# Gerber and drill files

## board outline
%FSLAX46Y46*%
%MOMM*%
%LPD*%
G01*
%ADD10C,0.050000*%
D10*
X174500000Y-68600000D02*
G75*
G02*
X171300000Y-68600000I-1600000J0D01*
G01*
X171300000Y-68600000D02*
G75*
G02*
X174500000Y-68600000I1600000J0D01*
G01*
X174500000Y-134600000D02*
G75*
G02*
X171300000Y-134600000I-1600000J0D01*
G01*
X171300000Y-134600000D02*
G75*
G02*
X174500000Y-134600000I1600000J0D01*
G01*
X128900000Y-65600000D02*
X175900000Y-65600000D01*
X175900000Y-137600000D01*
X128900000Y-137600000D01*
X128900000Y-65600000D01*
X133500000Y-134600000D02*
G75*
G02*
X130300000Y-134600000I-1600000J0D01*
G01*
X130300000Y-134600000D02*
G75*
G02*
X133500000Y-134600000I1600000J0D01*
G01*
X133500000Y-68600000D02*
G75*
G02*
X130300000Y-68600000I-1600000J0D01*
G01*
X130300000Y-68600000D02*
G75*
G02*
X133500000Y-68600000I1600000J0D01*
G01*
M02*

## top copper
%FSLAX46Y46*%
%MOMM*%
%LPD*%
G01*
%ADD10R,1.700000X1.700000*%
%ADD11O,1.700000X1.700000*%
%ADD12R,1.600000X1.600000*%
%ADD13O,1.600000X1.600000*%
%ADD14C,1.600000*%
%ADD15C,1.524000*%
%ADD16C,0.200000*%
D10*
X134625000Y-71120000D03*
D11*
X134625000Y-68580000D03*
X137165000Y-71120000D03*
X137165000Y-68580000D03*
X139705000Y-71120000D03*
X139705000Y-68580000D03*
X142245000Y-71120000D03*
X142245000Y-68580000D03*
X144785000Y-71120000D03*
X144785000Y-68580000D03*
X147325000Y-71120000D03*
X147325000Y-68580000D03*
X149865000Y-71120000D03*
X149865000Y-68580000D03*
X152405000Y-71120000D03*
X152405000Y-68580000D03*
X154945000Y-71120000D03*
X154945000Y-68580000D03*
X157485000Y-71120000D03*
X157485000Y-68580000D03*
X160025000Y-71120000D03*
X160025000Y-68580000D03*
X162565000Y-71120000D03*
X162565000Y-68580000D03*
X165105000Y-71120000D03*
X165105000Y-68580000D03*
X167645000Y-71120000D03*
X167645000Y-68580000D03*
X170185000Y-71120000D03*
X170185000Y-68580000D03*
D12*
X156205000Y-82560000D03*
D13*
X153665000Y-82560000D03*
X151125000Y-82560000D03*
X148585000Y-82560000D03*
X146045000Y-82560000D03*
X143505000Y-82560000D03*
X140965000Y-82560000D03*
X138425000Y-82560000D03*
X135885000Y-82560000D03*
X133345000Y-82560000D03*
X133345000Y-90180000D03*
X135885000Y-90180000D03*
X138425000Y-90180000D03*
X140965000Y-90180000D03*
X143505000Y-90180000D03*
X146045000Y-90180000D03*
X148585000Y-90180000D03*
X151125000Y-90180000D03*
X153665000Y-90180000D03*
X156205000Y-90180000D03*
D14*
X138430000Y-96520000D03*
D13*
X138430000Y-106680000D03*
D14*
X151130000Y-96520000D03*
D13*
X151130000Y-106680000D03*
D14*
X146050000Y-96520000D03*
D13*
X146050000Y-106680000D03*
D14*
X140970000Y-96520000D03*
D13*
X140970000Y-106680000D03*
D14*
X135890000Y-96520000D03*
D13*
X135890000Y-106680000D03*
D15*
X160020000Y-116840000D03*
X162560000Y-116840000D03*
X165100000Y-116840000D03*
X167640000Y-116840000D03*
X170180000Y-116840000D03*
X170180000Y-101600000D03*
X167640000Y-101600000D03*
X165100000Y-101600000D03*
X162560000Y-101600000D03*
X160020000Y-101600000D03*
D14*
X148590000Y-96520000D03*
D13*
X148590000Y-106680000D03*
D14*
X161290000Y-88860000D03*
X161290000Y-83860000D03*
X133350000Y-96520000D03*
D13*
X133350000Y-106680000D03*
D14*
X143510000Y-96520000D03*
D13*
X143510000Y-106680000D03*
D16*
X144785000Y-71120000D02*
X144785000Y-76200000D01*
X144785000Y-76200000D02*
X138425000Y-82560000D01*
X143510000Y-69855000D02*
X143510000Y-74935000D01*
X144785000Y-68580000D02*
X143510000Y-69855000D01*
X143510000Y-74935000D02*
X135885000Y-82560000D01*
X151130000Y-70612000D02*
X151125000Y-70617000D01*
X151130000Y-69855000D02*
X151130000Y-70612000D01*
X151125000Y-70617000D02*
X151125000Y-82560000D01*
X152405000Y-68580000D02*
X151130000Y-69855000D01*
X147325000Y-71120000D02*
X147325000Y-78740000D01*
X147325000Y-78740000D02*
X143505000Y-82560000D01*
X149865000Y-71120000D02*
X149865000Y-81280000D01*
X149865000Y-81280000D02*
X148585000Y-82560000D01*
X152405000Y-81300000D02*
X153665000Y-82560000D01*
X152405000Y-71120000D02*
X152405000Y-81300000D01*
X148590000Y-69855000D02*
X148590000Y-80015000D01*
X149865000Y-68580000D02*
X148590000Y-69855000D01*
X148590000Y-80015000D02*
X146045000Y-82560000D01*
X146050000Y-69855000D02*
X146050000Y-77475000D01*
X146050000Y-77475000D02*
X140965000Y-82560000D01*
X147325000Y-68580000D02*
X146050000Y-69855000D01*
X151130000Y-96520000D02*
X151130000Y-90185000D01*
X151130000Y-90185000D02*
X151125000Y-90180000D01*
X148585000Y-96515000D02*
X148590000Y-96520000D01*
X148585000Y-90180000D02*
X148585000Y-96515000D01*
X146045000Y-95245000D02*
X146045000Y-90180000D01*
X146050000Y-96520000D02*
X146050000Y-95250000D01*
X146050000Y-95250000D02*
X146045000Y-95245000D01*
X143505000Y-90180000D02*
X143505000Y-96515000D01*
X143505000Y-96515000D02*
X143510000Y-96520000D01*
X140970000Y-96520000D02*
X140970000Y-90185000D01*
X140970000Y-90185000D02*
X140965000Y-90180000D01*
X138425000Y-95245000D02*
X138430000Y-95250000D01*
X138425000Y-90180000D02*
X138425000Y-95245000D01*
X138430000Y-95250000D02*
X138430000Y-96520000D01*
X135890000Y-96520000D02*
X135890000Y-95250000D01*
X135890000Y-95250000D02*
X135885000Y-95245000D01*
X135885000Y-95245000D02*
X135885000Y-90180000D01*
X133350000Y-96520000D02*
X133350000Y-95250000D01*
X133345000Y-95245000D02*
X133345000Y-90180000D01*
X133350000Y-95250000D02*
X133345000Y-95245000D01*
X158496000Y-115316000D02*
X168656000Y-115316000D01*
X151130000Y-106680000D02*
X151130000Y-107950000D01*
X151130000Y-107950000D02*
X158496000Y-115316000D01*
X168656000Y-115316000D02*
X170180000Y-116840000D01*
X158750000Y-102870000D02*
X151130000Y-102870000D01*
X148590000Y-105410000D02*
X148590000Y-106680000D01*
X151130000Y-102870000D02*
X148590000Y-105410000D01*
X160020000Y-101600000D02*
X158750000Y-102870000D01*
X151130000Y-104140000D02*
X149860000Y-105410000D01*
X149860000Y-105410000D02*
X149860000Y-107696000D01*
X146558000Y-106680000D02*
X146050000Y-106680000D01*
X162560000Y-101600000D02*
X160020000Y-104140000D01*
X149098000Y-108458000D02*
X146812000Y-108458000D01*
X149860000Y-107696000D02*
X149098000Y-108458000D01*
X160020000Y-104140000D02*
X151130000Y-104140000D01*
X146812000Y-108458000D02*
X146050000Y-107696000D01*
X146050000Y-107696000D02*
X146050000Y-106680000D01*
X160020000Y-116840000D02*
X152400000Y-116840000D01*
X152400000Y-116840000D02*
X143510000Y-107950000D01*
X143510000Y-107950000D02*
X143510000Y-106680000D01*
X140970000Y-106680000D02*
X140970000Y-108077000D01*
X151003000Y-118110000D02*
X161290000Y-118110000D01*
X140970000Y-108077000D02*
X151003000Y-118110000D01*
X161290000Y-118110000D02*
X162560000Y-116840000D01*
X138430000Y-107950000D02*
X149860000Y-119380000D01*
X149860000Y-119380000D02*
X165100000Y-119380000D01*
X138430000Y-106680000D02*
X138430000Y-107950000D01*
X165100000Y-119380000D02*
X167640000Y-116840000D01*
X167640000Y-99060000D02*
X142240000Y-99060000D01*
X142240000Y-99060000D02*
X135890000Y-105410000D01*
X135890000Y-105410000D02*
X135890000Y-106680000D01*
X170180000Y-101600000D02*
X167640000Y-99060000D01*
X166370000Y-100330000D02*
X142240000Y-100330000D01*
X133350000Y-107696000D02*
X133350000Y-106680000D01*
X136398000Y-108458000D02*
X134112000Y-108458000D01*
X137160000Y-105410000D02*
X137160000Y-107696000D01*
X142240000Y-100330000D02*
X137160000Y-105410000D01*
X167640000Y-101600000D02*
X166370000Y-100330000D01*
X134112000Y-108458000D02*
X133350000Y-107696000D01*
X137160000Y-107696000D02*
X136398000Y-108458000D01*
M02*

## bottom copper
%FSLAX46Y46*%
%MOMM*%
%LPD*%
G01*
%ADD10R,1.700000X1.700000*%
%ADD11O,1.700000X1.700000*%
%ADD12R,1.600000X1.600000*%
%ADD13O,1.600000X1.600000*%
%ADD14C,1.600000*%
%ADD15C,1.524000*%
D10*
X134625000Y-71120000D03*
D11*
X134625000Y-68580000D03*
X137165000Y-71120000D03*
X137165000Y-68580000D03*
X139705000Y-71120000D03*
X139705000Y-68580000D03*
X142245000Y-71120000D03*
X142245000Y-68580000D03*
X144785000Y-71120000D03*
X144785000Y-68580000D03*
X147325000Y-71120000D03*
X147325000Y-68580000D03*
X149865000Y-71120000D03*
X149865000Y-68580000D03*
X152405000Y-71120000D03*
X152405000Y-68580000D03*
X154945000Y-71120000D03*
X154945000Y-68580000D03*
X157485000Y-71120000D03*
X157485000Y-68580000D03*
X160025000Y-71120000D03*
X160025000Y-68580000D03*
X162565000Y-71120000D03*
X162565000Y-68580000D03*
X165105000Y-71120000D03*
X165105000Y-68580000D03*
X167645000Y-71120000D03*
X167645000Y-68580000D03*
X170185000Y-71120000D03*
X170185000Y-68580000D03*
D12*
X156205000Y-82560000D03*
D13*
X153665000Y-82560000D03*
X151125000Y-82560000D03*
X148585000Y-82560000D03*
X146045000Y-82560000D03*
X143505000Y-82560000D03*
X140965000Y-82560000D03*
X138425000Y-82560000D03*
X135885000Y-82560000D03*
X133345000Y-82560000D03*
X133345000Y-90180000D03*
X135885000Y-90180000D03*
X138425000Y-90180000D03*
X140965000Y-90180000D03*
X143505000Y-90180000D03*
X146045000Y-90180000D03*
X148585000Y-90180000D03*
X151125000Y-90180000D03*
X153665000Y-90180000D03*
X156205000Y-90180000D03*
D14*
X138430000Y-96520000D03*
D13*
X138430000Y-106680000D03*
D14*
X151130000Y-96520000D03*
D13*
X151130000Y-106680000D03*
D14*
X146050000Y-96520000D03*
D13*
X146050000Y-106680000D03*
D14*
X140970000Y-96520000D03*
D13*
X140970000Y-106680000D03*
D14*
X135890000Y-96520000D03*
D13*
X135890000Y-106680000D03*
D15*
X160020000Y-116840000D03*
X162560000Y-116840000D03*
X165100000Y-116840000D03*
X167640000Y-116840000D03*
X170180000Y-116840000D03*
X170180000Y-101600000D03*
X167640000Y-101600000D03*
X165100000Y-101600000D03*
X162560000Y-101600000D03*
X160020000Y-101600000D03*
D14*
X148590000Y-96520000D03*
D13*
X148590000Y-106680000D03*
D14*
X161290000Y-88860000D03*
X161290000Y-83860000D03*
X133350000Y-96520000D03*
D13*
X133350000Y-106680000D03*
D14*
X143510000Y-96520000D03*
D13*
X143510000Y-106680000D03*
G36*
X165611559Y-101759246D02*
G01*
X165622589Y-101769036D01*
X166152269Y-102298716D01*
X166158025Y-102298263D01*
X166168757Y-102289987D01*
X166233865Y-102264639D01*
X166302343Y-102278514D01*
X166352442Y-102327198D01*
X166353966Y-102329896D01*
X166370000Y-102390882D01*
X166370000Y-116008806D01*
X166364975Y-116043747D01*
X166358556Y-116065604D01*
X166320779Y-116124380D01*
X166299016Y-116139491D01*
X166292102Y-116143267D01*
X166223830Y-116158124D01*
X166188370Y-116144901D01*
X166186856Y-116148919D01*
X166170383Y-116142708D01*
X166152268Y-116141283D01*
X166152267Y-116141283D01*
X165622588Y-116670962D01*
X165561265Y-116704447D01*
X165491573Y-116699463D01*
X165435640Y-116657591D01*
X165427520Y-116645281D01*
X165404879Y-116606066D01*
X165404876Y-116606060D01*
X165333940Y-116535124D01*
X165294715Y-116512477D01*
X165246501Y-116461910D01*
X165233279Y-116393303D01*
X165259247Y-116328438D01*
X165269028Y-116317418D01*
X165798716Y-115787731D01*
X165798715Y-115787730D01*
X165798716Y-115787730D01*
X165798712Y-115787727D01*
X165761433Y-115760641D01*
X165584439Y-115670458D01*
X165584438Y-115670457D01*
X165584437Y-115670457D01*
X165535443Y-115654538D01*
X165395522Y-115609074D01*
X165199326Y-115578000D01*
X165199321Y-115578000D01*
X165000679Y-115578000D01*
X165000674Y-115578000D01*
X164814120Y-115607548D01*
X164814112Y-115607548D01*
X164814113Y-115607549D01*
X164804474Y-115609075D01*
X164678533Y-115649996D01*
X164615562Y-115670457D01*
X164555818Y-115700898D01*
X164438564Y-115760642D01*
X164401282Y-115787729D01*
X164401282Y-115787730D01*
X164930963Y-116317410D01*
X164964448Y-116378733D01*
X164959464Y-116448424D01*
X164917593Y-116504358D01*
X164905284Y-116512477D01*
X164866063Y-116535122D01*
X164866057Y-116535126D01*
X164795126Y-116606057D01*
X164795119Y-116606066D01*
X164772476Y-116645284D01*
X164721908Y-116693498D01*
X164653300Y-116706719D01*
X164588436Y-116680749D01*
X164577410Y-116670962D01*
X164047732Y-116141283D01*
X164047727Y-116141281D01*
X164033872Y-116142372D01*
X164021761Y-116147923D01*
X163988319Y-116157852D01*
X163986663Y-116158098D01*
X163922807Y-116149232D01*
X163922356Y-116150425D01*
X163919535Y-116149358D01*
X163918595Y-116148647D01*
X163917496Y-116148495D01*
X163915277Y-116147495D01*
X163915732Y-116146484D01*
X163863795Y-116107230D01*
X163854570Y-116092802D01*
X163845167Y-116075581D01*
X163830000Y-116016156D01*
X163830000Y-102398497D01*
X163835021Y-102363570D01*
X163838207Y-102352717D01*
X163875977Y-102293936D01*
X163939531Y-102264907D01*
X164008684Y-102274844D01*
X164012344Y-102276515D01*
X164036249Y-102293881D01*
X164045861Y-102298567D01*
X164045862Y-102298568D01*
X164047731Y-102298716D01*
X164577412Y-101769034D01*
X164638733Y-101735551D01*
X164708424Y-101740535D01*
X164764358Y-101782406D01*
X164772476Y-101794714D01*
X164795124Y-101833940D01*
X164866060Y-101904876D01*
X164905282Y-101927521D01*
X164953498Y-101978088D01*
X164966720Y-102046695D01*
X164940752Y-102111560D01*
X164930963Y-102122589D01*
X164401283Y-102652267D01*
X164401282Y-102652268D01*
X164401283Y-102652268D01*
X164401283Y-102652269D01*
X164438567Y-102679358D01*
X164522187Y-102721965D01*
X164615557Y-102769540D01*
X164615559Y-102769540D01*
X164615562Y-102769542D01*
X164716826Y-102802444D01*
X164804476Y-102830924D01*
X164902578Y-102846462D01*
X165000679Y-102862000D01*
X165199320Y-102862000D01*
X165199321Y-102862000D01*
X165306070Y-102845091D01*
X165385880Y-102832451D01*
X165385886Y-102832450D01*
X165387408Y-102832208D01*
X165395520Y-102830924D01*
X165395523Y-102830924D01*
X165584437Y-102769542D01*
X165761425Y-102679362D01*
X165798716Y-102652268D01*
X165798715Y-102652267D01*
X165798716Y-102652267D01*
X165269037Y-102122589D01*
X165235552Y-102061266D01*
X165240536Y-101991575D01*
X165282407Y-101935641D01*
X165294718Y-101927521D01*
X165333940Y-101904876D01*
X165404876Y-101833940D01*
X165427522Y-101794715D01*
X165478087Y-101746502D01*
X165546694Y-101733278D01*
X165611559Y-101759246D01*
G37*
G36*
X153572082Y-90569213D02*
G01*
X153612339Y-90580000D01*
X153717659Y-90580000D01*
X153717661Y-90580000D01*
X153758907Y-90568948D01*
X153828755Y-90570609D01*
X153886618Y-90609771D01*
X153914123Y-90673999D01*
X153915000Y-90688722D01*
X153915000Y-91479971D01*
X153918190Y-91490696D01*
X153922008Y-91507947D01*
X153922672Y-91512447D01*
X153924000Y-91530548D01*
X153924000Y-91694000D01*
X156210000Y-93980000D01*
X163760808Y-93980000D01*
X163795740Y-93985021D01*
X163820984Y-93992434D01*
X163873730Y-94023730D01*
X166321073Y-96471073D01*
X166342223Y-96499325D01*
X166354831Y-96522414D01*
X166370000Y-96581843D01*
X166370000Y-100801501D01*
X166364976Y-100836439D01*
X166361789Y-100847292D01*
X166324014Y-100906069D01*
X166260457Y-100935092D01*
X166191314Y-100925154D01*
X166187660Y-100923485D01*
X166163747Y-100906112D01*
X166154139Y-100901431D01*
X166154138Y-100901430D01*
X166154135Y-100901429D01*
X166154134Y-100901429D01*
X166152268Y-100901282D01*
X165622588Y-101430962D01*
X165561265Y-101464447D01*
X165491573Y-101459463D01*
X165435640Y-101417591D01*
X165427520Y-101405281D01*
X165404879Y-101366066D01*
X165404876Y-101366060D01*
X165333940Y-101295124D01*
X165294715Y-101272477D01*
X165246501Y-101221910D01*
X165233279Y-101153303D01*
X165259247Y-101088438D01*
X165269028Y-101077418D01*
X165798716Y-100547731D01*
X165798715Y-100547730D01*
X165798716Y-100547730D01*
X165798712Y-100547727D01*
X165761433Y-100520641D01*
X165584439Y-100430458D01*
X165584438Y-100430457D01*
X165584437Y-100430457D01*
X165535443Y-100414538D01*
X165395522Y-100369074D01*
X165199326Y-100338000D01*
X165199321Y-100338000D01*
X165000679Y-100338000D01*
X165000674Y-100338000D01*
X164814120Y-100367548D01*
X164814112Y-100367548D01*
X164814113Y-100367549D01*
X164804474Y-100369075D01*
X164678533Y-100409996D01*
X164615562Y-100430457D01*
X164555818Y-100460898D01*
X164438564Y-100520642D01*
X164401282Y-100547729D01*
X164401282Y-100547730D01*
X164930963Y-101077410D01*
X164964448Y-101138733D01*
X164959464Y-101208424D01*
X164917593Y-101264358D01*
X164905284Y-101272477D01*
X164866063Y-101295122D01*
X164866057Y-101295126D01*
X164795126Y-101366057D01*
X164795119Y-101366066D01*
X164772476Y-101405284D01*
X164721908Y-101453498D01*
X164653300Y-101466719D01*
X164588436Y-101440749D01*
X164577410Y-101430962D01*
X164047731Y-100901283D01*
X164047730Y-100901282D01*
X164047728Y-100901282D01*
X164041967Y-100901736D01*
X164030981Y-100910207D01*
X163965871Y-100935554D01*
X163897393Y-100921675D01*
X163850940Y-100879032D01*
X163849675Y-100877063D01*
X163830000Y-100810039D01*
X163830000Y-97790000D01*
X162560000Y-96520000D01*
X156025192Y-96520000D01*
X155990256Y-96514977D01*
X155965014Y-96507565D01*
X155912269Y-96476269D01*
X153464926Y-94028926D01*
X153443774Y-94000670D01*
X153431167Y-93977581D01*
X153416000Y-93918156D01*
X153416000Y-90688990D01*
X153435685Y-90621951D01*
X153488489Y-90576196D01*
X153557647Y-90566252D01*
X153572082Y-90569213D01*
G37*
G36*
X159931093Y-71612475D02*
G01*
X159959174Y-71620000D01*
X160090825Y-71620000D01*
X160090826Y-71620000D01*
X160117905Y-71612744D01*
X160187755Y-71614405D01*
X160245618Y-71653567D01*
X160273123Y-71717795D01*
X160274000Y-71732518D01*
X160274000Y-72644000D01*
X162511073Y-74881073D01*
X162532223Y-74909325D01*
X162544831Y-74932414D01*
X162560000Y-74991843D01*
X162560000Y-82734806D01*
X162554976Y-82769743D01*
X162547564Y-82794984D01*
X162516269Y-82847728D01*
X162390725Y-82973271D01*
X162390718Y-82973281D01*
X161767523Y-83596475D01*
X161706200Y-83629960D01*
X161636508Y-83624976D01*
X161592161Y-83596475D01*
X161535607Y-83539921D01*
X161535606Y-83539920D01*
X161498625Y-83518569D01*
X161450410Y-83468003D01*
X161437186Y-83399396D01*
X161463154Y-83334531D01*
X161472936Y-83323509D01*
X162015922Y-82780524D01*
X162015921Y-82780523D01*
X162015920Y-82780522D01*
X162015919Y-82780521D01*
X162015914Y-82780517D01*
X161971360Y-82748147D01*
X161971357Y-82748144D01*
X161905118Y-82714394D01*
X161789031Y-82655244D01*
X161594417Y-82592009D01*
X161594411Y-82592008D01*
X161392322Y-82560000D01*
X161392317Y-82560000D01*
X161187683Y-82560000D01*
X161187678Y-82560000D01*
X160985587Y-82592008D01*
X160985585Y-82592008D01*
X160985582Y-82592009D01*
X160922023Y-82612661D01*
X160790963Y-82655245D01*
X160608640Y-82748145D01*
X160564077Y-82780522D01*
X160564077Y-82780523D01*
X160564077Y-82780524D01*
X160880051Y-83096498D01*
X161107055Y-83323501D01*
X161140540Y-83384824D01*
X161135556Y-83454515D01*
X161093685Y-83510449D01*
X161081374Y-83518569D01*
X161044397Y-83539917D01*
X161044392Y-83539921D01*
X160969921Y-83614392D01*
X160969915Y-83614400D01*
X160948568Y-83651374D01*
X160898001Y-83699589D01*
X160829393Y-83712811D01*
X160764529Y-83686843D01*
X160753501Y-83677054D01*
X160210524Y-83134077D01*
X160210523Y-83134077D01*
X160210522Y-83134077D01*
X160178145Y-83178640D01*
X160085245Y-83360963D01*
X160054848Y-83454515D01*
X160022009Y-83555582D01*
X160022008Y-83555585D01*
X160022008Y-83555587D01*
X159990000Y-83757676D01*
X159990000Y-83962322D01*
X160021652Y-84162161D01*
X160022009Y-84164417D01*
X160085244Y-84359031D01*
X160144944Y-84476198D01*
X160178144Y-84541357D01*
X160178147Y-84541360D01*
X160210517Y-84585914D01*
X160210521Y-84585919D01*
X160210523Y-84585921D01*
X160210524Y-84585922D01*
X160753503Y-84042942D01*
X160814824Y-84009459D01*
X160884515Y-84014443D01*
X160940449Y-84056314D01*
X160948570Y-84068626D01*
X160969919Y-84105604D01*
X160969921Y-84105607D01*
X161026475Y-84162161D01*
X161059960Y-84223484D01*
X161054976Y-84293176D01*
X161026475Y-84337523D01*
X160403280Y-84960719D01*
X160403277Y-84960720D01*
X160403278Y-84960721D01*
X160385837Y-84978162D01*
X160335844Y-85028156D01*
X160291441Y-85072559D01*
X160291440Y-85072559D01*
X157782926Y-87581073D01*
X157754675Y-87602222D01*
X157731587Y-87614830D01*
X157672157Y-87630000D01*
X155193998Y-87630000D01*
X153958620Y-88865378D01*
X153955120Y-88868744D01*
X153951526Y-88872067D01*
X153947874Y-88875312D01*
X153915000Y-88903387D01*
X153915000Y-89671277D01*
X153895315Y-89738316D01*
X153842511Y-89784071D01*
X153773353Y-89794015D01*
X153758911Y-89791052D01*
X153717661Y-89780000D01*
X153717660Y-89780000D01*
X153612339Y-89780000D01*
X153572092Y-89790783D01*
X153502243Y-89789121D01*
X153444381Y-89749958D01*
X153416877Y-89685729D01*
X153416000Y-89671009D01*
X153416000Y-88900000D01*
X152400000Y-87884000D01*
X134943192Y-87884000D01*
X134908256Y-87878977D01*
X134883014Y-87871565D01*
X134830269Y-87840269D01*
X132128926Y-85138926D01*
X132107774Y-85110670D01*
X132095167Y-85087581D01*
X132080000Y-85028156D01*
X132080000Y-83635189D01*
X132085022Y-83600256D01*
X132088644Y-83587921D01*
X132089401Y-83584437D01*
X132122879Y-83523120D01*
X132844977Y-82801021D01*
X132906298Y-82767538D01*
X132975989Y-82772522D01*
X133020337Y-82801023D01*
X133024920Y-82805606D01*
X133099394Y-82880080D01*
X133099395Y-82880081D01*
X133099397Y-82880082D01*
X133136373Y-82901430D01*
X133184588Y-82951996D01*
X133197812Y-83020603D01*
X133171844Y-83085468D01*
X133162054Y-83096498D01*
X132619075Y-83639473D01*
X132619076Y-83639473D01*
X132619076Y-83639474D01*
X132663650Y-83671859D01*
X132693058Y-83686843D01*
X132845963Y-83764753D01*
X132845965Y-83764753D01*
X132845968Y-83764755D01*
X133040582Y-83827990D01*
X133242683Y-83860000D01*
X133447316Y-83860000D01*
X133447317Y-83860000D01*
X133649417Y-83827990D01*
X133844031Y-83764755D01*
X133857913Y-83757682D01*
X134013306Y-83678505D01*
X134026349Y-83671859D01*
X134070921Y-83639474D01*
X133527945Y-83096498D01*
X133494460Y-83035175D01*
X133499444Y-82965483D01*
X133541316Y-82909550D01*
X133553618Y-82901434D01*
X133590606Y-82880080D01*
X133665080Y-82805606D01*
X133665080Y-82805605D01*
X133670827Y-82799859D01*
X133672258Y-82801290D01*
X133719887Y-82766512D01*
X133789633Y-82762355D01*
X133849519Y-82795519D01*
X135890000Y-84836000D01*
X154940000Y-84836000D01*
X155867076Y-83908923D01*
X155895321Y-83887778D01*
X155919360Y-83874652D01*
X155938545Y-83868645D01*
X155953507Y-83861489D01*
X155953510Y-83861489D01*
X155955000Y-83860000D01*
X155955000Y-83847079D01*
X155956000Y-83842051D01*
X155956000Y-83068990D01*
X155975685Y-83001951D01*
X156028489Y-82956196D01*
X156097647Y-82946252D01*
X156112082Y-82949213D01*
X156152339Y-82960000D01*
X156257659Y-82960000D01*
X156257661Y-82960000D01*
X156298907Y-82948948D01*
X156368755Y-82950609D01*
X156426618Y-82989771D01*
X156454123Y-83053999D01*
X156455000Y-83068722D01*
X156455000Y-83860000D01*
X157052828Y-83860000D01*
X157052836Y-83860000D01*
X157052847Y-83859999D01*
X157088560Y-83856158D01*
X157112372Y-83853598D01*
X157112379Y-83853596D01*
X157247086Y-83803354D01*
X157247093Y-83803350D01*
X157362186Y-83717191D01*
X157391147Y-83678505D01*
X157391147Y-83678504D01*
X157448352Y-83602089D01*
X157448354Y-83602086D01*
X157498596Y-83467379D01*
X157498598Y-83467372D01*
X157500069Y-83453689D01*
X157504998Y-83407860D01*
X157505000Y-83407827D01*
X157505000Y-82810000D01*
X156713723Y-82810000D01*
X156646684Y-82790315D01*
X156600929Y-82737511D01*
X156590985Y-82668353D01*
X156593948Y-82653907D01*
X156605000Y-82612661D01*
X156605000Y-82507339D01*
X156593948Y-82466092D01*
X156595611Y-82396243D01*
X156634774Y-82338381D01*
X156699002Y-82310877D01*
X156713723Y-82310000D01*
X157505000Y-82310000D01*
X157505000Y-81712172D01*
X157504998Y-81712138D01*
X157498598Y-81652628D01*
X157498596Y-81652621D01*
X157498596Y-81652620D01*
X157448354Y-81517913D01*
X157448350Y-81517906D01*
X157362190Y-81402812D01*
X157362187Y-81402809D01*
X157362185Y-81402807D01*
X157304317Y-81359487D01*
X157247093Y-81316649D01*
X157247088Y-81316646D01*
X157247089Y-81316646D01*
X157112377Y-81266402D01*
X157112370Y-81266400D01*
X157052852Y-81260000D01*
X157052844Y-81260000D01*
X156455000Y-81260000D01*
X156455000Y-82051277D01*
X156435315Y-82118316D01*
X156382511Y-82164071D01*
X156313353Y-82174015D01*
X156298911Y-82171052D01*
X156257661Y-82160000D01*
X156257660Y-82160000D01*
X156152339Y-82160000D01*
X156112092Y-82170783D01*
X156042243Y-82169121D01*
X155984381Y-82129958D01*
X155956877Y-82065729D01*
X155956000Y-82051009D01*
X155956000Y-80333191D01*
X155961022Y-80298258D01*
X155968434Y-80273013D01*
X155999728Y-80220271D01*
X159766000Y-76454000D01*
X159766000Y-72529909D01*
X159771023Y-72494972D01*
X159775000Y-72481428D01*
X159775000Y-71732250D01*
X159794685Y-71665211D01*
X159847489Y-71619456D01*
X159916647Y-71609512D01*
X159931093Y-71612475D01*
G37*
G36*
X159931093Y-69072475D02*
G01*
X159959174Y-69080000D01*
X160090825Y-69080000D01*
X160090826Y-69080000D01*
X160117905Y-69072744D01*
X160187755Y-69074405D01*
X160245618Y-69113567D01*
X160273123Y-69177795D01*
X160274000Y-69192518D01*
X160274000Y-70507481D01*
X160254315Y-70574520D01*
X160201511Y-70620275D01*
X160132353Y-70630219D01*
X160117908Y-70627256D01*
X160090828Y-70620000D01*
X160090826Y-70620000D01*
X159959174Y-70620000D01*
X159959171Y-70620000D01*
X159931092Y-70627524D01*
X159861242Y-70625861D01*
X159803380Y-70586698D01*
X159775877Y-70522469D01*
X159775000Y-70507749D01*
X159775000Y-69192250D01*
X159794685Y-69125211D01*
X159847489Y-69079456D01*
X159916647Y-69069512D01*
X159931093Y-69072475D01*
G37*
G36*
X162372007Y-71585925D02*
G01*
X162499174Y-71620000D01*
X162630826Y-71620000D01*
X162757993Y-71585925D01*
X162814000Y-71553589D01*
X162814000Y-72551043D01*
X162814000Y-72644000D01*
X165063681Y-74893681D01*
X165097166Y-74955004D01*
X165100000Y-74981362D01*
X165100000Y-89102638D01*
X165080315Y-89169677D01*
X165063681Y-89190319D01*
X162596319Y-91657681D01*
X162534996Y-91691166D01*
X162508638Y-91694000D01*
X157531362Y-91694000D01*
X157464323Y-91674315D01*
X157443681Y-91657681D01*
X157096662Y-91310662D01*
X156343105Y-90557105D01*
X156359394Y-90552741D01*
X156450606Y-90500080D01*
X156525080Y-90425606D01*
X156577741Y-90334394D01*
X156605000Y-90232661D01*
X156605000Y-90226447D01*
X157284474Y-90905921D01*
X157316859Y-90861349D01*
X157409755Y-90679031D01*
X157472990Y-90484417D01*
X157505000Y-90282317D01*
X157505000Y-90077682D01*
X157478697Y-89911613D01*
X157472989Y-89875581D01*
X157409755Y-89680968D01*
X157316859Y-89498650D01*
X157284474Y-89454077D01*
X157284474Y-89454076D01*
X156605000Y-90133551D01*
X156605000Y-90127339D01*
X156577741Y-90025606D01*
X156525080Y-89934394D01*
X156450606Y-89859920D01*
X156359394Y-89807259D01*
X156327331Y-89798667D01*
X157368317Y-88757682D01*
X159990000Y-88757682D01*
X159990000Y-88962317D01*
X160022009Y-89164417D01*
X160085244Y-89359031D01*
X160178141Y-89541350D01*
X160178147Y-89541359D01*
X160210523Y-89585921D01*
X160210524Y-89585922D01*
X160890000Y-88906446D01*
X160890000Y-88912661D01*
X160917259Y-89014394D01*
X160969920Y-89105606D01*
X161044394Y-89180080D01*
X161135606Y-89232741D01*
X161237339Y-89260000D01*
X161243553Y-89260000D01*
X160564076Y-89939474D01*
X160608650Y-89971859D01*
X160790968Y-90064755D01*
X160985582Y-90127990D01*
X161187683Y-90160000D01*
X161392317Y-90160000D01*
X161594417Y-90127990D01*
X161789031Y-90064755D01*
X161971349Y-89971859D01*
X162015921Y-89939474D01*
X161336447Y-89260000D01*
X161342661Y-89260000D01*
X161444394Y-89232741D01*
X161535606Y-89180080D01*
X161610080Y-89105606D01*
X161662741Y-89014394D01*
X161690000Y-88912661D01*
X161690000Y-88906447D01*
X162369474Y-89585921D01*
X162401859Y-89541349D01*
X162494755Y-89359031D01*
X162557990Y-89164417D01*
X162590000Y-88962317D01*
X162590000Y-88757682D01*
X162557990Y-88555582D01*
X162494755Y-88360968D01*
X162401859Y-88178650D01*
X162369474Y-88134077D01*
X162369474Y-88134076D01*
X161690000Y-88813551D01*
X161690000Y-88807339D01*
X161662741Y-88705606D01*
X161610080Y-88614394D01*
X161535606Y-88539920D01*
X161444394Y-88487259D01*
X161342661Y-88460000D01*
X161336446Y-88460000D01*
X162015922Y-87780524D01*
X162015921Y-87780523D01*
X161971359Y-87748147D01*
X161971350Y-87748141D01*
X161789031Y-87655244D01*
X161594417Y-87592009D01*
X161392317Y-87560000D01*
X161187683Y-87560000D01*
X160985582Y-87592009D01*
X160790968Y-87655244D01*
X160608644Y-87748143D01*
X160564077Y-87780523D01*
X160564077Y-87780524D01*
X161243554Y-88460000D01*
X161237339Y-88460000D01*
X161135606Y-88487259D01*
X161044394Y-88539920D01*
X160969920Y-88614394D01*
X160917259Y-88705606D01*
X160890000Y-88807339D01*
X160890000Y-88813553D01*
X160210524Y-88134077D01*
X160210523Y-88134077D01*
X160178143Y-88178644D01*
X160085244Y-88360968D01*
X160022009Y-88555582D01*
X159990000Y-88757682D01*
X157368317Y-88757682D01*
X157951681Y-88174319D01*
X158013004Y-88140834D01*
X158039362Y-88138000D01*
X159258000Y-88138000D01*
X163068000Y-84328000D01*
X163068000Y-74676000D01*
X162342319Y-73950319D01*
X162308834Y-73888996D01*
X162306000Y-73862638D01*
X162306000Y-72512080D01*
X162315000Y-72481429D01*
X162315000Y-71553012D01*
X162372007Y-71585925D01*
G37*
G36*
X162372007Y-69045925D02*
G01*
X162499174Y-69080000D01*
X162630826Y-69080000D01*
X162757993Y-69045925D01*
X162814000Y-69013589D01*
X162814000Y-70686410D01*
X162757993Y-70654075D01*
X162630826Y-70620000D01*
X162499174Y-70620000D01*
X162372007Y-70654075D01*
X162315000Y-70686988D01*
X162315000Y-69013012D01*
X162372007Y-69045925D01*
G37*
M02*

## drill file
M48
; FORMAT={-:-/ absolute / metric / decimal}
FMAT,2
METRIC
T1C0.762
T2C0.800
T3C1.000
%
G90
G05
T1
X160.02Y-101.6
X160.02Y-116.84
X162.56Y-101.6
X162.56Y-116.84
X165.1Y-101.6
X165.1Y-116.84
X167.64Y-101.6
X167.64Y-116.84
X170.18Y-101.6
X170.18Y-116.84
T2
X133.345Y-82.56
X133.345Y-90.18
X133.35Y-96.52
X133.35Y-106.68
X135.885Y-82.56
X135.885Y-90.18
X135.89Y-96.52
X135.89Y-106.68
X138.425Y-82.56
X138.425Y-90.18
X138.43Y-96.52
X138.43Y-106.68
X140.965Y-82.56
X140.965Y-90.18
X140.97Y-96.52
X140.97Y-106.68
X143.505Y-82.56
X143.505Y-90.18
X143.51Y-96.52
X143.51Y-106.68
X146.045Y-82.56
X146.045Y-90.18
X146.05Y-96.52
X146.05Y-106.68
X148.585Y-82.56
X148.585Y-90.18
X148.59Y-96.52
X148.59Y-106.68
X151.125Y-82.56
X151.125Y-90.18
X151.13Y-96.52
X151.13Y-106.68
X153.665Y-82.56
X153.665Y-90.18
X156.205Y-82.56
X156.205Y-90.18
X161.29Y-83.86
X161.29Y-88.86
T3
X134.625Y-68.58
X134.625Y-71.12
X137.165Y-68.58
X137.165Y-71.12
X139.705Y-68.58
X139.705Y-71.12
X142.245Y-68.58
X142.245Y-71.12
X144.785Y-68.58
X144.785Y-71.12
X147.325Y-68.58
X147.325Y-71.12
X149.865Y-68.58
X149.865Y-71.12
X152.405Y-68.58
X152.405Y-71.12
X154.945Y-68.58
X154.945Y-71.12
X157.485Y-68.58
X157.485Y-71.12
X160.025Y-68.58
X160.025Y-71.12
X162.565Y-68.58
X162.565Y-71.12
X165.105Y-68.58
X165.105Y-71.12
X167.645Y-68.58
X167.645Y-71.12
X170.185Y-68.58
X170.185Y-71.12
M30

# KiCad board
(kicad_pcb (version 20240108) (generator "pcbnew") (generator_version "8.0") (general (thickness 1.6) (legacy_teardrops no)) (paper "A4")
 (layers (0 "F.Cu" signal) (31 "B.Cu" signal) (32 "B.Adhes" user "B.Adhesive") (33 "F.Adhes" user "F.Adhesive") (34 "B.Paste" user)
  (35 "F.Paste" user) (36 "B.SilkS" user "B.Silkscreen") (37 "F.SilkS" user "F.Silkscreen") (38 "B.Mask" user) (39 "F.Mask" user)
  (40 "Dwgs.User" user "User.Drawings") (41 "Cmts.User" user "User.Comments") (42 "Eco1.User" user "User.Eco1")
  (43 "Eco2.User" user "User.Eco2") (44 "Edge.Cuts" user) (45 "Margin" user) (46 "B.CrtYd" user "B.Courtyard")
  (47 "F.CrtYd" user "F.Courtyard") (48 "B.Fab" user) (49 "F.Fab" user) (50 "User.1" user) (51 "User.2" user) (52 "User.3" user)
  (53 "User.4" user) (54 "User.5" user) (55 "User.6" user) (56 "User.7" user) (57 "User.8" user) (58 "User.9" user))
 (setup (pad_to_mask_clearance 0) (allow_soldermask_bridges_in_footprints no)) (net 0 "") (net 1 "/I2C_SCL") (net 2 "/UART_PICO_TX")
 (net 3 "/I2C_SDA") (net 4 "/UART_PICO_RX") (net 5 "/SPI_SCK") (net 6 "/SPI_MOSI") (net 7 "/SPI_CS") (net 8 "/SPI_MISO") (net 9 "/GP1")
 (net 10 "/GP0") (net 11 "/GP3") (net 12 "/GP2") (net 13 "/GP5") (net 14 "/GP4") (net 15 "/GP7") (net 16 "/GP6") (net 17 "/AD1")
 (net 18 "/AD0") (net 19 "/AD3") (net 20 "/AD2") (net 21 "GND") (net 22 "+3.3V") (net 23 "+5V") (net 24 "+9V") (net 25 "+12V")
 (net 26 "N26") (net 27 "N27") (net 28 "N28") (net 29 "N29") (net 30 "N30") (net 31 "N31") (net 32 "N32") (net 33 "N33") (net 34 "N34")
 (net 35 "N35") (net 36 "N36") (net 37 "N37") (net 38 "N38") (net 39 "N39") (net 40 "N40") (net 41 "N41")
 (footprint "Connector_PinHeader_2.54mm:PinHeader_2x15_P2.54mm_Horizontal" (layer "F.Cu") (at 134.625 71.12 90)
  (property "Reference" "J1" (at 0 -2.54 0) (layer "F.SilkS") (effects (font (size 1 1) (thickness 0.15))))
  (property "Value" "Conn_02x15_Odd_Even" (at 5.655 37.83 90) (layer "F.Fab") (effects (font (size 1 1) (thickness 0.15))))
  (pad "1" thru_hole rect (at 0 0 90) (size 1.7 1.7) (drill 1) (layers "*.Cu" "*.Mask") (remove_unused_layers no) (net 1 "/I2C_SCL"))
  (pad "2" thru_hole oval (at 2.54 0 90) (size 1.7 1.7) (drill 1) (layers "*.Cu" "*.Mask") (remove_unused_layers no) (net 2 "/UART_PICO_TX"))
  (pad "3" thru_hole oval (at 0 2.54 90) (size 1.7 1.7) (drill 1) (layers "*.Cu" "*.Mask") (remove_unused_layers no) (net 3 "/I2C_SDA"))
  (pad "4" thru_hole oval (at 2.54 2.54 90) (size 1.7 1.7) (drill 1) (layers "*.Cu" "*.Mask") (remove_unused_layers no)
   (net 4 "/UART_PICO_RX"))
  (pad "5" thru_hole oval (at 0 5.08 90) (size 1.7 1.7) (drill 1) (layers "*.Cu" "*.Mask") (remove_unused_layers no) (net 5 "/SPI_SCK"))
  (pad "6" thru_hole oval (at 2.54 5.08 90) (size 1.7 1.7) (drill 1) (layers "*.Cu" "*.Mask") (remove_unused_layers no) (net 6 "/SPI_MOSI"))
  (pad "7" thru_hole oval (at 0 7.62 90) (size 1.7 1.7) (drill 1) (layers "*.Cu" "*.Mask") (remove_unused_layers no) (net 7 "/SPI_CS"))
  (pad "8" thru_hole oval (at 2.54 7.62 90) (size 1.7 1.7) (drill 1) (layers "*.Cu" "*.Mask") (remove_unused_layers no) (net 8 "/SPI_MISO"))
  (pad "9" thru_hole oval (at 0 10.16 90) (size 1.7 1.7) (drill 1) (layers "*.Cu" "*.Mask") (remove_unused_layers no) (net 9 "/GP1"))
  (pad "10" thru_hole oval (at 2.54 10.16 90) (size 1.7 1.7) (drill 1) (layers "*.Cu" "*.Mask") (remove_unused_layers no) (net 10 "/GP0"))
  (pad "11" thru_hole oval (at 0 12.7 90) (size 1.7 1.7) (drill 1) (layers "*.Cu" "*.Mask") (remove_unused_layers no) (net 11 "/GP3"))
  (pad "12" thru_hole oval (at 2.54 12.7 90) (size 1.7 1.7) (drill 1) (layers "*.Cu" "*.Mask") (remove_unused_layers no) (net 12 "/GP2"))
  (pad "13" thru_hole oval (at 0 15.24 90) (size 1.7 1.7) (drill 1) (layers "*.Cu" "*.Mask") (remove_unused_layers no) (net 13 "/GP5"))
  (pad "14" thru_hole oval (at 2.54 15.24 90) (size 1.7 1.7) (drill 1) (layers "*.Cu" "*.Mask") (remove_unused_layers no) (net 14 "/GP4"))
  (pad "15" thru_hole oval (at 0 17.78 90) (size 1.7 1.7) (drill 1) (layers "*.Cu" "*.Mask") (remove_unused_layers no) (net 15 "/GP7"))
  (pad "16" thru_hole oval (at 2.54 17.78 90) (size 1.7 1.7) (drill 1) (layers "*.Cu" "*.Mask") (remove_unused_layers no) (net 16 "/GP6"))
  (pad "17" thru_hole oval (at 0 20.32 90) (size 1.7 1.7) (drill 1) (layers "*.Cu" "*.Mask") (remove_unused_layers no) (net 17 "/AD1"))
  (pad "18" thru_hole oval (at 2.54 20.32 90) (size 1.7 1.7) (drill 1) (layers "*.Cu" "*.Mask") (remove_unused_layers no) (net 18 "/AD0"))
  (pad "19" thru_hole oval (at 0 22.86 90) (size 1.7 1.7) (drill 1) (layers "*.Cu" "*.Mask") (remove_unused_layers no) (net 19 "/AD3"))
  (pad "20" thru_hole oval (at 2.54 22.86 90) (size 1.7 1.7) (drill 1) (layers "*.Cu" "*.Mask") (remove_unused_layers no) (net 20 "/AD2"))
  (pad "21" thru_hole oval (at 0 25.4 90) (size 1.7 1.7) (drill 1) (layers "*.Cu" "*.Mask") (remove_unused_layers no) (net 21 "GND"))
  (pad "22" thru_hole oval (at 2.54 25.4 90) (size 1.7 1.7) (drill 1) (layers "*.Cu" "*.Mask") (remove_unused_layers no) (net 21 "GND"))
  (pad "23" thru_hole oval (at 0 27.94 90) (size 1.7 1.7) (drill 1) (layers "*.Cu" "*.Mask") (remove_unused_layers no) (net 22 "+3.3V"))
  (pad "24" thru_hole oval (at 2.54 27.94 90) (size 1.7 1.7) (drill 1) (layers "*.Cu" "*.Mask") (remove_unused_layers no) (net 22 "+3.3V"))
  (pad "25" thru_hole oval (at 0 30.48 90) (size 1.7 1.7) (drill 1) (layers "*.Cu" "*.Mask") (remove_unused_layers no) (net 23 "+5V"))
  (pad "26" thru_hole oval (at 2.54 30.48 90) (size 1.7 1.7) (drill 1) (layers "*.Cu" "*.Mask") (remove_unused_layers no) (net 23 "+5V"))
  (pad "27" thru_hole oval (at 0 33.02 90) (size 1.7 1.7) (drill 1) (layers "*.Cu" "*.Mask") (remove_unused_layers no) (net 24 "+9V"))
  (pad "28" thru_hole oval (at 2.54 33.02 90) (size 1.7 1.7) (drill 1) (layers "*.Cu" "*.Mask") (remove_unused_layers no) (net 24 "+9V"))
  (pad "29" thru_hole oval (at 0 35.56 90) (size 1.7 1.7) (drill 1) (layers "*.Cu" "*.Mask") (remove_unused_layers no) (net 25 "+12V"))
  (pad "30" thru_hole oval (at 2.54 35.56 90) (size 1.7 1.7) (drill 1) (layers "*.Cu" "*.Mask") (remove_unused_layers no) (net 25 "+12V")))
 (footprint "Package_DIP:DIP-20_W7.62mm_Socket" (layer "F.Cu") (at 156.205 82.56 -90)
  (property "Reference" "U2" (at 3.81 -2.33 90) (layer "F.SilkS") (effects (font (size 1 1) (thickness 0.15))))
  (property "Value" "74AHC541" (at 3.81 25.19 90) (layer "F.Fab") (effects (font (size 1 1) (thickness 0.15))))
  (pad "1" thru_hole rect (at 0 0 270) (size 1.6 1.6) (drill 0.8) (layers "*.Cu" "*.Mask") (remove_unused_layers no) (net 21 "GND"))
  (pad "2" thru_hole oval (at 0 2.54 270) (size 1.6 1.6) (drill 0.8) (layers "*.Cu" "*.Mask") (remove_unused_layers no) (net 15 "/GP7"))
  (pad "3" thru_hole oval (at 0 5.08 270) (size 1.6 1.6) (drill 0.8) (layers "*.Cu" "*.Mask") (remove_unused_layers no) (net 16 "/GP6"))
  (pad "4" thru_hole oval (at 0 7.62 270) (size 1.6 1.6) (drill 0.8) (layers "*.Cu" "*.Mask") (remove_unused_layers no) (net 13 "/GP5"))
  (pad "5" thru_hole oval (at 0 10.16 270) (size 1.6 1.6) (drill 0.8) (layers "*.Cu" "*.Mask") (remove_unused_layers no) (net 14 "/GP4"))
  (pad "6" thru_hole oval (at 0 12.7 270) (size 1.6 1.6) (drill 0.8) (layers "*.Cu" "*.Mask") (remove_unused_layers no) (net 11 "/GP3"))
  (pad "7" thru_hole oval (at 0 15.24 270) (size 1.6 1.6) (drill 0.8) (layers "*.Cu" "*.Mask") (remove_unused_layers no) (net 12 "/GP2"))
  (pad "8" thru_hole oval (at 0 17.78 270) (size 1.6 1.6) (drill 0.8) (layers "*.Cu" "*.Mask") (remove_unused_layers no) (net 9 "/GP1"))
  (pad "9" thru_hole oval (at 0 20.32 270) (size 1.6 1.6) (drill 0.8) (layers "*.Cu" "*.Mask") (remove_unused_layers no) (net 10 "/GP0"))
  (pad "10" thru_hole oval (at 0 22.86 270) (size 1.6 1.6) (drill 0.8) (layers "*.Cu" "*.Mask") (remove_unused_layers no) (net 21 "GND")
   (thermal_bridge_angle 45))
  (pad "11" thru_hole oval (at 7.62 22.86 270) (size 1.6 1.6) (drill 0.8) (layers "*.Cu" "*.Mask") (remove_unused_layers no) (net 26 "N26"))
  (pad "12" thru_hole oval (at 7.62 20.32 270) (size 1.6 1.6) (drill 0.8) (layers "*.Cu" "*.Mask") (remove_unused_layers no) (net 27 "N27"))
  (pad "13" thru_hole oval (at 7.62 17.78 270) (size 1.6 1.6) (drill 0.8) (layers "*.Cu" "*.Mask") (remove_unused_layers no) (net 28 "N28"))
  (pad "14" thru_hole oval (at 7.62 15.24 270) (size 1.6 1.6) (drill 0.8) (layers "*.Cu" "*.Mask") (remove_unused_layers no) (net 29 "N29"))
  (pad "15" thru_hole oval (at 7.62 12.7 270) (size 1.6 1.6) (drill 0.8) (layers "*.Cu" "*.Mask") (remove_unused_layers no) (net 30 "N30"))
  (pad "16" thru_hole oval (at 7.62 10.16 270) (size 1.6 1.6) (drill 0.8) (layers "*.Cu" "*.Mask") (remove_unused_layers no) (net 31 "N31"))
  (pad "17" thru_hole oval (at 7.62 7.62 270) (size 1.6 1.6) (drill 0.8) (layers "*.Cu" "*.Mask") (remove_unused_layers no) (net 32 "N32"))
  (pad "18" thru_hole oval (at 7.62 5.08 270) (size 1.6 1.6) (drill 0.8) (layers "*.Cu" "*.Mask") (remove_unused_layers no) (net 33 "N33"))
  (pad "19" thru_hole oval (at 7.62 2.54 270) (size 1.6 1.6) (drill 0.8) (layers "*.Cu" "*.Mask") (remove_unused_layers no) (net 21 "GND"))
  (pad "20" thru_hole oval (at 7.62 0 270) (size 1.6 1.6) (drill 0.8) (layers "*.Cu" "*.Mask") (remove_unused_layers no) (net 22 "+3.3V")
   (thermal_bridge_angle 45)))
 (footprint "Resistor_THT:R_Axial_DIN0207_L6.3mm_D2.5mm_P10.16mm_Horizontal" (layer "F.Cu") (at 138.43 96.52 -90)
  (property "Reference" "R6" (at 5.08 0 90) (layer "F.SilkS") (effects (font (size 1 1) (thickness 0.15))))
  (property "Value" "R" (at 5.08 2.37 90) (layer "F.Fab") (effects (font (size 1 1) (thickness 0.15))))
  (pad "1" thru_hole circle (at 0 0 270) (size 1.6 1.6) (drill 0.8) (layers "*.Cu" "*.Mask") (remove_unused_layers no) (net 28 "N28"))
  (pad "2" thru_hole oval (at 10.16 0 270) (size 1.6 1.6) (drill 0.8) (layers "*.Cu" "*.Mask") (remove_unused_layers no) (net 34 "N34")))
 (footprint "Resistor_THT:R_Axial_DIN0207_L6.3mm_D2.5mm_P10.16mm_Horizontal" (layer "F.Cu") (at 151.13 96.52 -90)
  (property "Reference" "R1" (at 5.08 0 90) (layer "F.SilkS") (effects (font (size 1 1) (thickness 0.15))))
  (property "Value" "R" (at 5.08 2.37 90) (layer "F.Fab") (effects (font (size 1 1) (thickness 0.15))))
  (pad "1" thru_hole circle (at 0 0 270) (size 1.6 1.6) (drill 0.8) (layers "*.Cu" "*.Mask") (remove_unused_layers no) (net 33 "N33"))
  (pad "2" thru_hole oval (at 10.16 0 270) (size 1.6 1.6) (drill 0.8) (layers "*.Cu" "*.Mask") (remove_unused_layers no) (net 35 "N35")))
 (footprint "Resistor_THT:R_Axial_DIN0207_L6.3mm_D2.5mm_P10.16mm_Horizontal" (layer "F.Cu") (at 146.05 96.52 -90)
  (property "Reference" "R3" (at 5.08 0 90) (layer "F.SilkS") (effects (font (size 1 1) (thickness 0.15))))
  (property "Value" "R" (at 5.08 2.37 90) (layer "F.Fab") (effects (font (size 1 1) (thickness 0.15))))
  (pad "1" thru_hole circle (at 0 0 270) (size 1.6 1.6) (drill 0.8) (layers "*.Cu" "*.Mask") (remove_unused_layers no) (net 31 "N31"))
  (pad "2" thru_hole oval (at 10.16 0 270) (size 1.6 1.6) (drill 0.8) (layers "*.Cu" "*.Mask") (remove_unused_layers no) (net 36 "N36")))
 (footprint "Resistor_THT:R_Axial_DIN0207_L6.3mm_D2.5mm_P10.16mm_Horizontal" (layer "F.Cu") (at 140.97 96.52 -90)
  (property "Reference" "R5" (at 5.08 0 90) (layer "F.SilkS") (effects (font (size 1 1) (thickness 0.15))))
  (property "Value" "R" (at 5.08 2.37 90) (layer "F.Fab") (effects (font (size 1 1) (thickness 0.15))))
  (pad "1" thru_hole circle (at 0 0 270) (size 1.6 1.6) (drill 0.8) (layers "*.Cu" "*.Mask") (remove_unused_layers no) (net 29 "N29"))
  (pad "2" thru_hole oval (at 10.16 0 270) (size 1.6 1.6) (drill 0.8) (layers "*.Cu" "*.Mask") (remove_unused_layers no) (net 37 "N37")))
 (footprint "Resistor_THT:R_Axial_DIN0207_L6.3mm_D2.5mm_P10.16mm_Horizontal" (layer "F.Cu") (at 135.89 96.52 -90)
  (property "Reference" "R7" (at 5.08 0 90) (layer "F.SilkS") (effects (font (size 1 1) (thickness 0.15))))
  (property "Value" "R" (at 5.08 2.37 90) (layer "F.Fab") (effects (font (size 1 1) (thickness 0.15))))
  (pad "1" thru_hole circle (at 0 0 270) (size 1.6 1.6) (drill 0.8) (layers "*.Cu" "*.Mask") (remove_unused_layers no) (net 27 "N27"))
  (pad "2" thru_hole oval (at 10.16 0 270) (size 1.6 1.6) (drill 0.8) (layers "*.Cu" "*.Mask") (remove_unused_layers no) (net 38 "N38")))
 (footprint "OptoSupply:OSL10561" (layer "F.Cu") (at 165.1 109.22)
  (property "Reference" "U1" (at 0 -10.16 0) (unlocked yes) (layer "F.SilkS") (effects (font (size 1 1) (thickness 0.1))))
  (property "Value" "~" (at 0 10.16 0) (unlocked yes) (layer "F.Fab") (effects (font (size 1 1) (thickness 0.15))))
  (pad "1" thru_hole circle (at -5.08 7.62) (size 1.524 1.524) (drill 0.762) (layers "*.Cu" "*.Mask") (remove_unused_layers no)
   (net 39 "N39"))
  (pad "2" thru_hole circle (at -2.54 7.62) (size 1.524 1.524) (drill 0.762) (layers "*.Cu" "*.Mask") (remove_unused_layers no)
   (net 37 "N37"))
  (pad "3" thru_hole circle (at 0 7.62) (size 1.524 1.524) (drill 0.762) (layers "*.Cu" "*.Mask") (remove_unused_layers no) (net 21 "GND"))
  (pad "4" thru_hole circle (at 2.54 7.62) (size 1.524 1.524) (drill 0.762) (layers "*.Cu" "*.Mask") (remove_unused_layers no)
   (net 34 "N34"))
  (pad "5" thru_hole circle (at 5.08 7.62) (size 1.524 1.524) (drill 0.762) (layers "*.Cu" "*.Mask") (remove_unused_layers no)
   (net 35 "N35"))
  (pad "6" thru_hole circle (at 5.08 -7.62) (size 1.524 1.524) (drill 0.762) (layers "*.Cu" "*.Mask") (remove_unused_layers no)
   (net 38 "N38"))
  (pad "7" thru_hole circle (at 2.54 -7.62) (size 1.524 1.524) (drill 0.762) (layers "*.Cu" "*.Mask") (remove_unused_layers no)
   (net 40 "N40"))
  (pad "8" thru_hole circle (at 0 -7.62) (size 1.524 1.524) (drill 0.762) (layers "*.Cu" "*.Mask") (remove_unused_layers no) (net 21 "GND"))
  (pad "9" thru_hole circle (at -2.54 -7.62) (size 1.524 1.524) (drill 0.762) (layers "*.Cu" "*.Mask") (remove_unused_layers no)
   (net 36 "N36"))
  (pad "10" thru_hole circle (at -5.08 -7.62) (size 1.524 1.524) (drill 0.762) (layers "*.Cu" "*.Mask") (remove_unused_layers no)
   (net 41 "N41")))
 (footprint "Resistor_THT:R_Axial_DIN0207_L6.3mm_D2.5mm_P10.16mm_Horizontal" (layer "F.Cu") (at 148.59 96.52 -90)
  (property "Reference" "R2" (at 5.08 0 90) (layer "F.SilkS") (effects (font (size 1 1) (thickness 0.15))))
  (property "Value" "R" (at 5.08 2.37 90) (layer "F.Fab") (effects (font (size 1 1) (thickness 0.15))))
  (pad "1" thru_hole circle (at 0 0 270) (size 1.6 1.6) (drill 0.8) (layers "*.Cu" "*.Mask") (remove_unused_layers no) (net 32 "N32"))
  (pad "2" thru_hole oval (at 10.16 0 270) (size 1.6 1.6) (drill 0.8) (layers "*.Cu" "*.Mask") (remove_unused_layers no) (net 41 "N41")))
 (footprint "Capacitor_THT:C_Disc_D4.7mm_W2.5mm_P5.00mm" (layer "F.Cu") (at 161.29 88.86 90)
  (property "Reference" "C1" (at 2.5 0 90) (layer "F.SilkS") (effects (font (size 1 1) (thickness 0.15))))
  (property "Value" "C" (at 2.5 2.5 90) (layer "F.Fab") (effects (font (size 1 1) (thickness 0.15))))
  (pad "1" thru_hole circle (at 0 0 90) (size 1.6 1.6) (drill 0.8) (layers "*.Cu" "*.Mask") (remove_unused_layers no) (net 22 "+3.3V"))
  (pad "2" thru_hole circle (at 5 0 90) (size 1.6 1.6) (drill 0.8) (layers "*.Cu" "*.Mask") (remove_unused_layers no) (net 21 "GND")))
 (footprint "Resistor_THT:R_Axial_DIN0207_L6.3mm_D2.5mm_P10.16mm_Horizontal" (layer "F.Cu") (at 133.35 96.52 -90)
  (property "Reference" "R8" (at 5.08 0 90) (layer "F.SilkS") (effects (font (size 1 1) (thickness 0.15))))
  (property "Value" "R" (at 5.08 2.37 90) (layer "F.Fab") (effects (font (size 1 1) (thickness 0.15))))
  (pad "1" thru_hole circle (at 0 0 270) (size 1.6 1.6) (drill 0.8) (layers "*.Cu" "*.Mask") (remove_unused_layers no) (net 26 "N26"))
  (pad "2" thru_hole oval (at 10.16 0 270) (size 1.6 1.6) (drill 0.8) (layers "*.Cu" "*.Mask") (remove_unused_layers no) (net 40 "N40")))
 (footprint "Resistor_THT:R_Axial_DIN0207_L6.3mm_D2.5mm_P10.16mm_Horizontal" (layer "F.Cu") (at 143.51 96.52 -90)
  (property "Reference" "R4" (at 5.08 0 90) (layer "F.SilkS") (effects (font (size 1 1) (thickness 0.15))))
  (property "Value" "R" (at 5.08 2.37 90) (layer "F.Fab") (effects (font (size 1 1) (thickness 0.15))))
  (pad "1" thru_hole circle (at 0 0 270) (size 1.6 1.6) (drill 0.8) (layers "*.Cu" "*.Mask") (remove_unused_layers no) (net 30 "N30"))
  (pad "2" thru_hole oval (at 10.16 0 270) (size 1.6 1.6) (drill 0.8) (layers "*.Cu" "*.Mask") (remove_unused_layers no) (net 39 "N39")))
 (gr_circle (center 172.9 68.6) (end 172.9 70.2) (stroke (width 0.05) (type default)) (fill none) (layer "Edge.Cuts"))
 (gr_circle (center 172.9 134.6) (end 171.3 134.6) (stroke (width 0.05) (type default)) (fill none) (layer "Edge.Cuts"))
 (gr_rect (start 128.9 65.6) (end 175.9 137.6) (stroke (width 0.05) (type default)) (fill none) (layer "Edge.Cuts"))
 (gr_circle (center 131.9 134.6) (end 131.9 133) (stroke (width 0.05) (type default)) (fill none) (layer "Edge.Cuts"))
 (gr_circle (center 131.9 68.6) (end 133.5 68.6) (stroke (width 0.05) (type default)) (fill none) (layer "Edge.Cuts"))
 (segment (start 144.785 71.12) (end 144.785 76.2) (width 0.2) (layer "F.Cu") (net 9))
 (segment (start 144.785 76.2) (end 138.425 82.56) (width 0.2) (layer "F.Cu") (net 9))
 (segment (start 143.51 69.855) (end 143.51 74.935) (width 0.2) (layer "F.Cu") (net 10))
 (segment (start 144.785 68.58) (end 143.51 69.855) (width 0.2) (layer "F.Cu") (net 10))
 (segment (start 143.51 74.935) (end 135.885 82.56) (width 0.2) (layer "F.Cu") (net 10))
 (segment (start 151.13 70.612) (end 151.125 70.617) (width 0.2) (layer "F.Cu") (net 16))
 (segment (start 151.13 69.855) (end 151.13 70.612) (width 0.2) (layer "F.Cu") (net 16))
 (segment (start 151.125 70.617) (end 151.125 82.56) (width 0.2) (layer "F.Cu") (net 16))
 (segment (start 152.405 68.58) (end 151.13 69.855) (width 0.2) (layer "F.Cu") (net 16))
 (segment (start 147.325 71.12) (end 147.325 78.74) (width 0.2) (layer "F.Cu") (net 11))
 (segment (start 147.325 78.74) (end 143.505 82.56) (width 0.2) (layer "F.Cu") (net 11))
 (segment (start 149.865 71.12) (end 149.865 81.28) (width 0.2) (layer "F.Cu") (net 13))
 (segment (start 149.865 81.28) (end 148.585 82.56) (width 0.2) (layer "F.Cu") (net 13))
 (segment (start 152.405 81.3) (end 153.665 82.56) (width 0.2) (layer "F.Cu") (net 15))
 (segment (start 152.405 71.12) (end 152.405 81.3) (width 0.2) (layer "F.Cu") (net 15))
 (segment (start 148.59 69.855) (end 148.59 80.015) (width 0.2) (layer "F.Cu") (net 14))
 (segment (start 149.865 68.58) (end 148.59 69.855) (width 0.2) (layer "F.Cu") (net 14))
 (segment (start 148.59 80.015) (end 146.045 82.56) (width 0.2) (layer "F.Cu") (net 14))
 (segment (start 146.05 69.855) (end 146.05 77.475) (width 0.2) (layer "F.Cu") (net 12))
 (segment (start 146.05 77.475) (end 140.965 82.56) (width 0.2) (layer "F.Cu") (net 12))
 (segment (start 147.325 68.58) (end 146.05 69.855) (width 0.2) (layer "F.Cu") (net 12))
 (segment (start 151.13 96.52) (end 151.13 90.185) (width 0.2) (layer "F.Cu") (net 33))
 (segment (start 151.13 90.185) (end 151.125 90.18) (width 0.2) (layer "F.Cu") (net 33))
 (segment (start 148.585 96.515) (end 148.59 96.52) (width 0.2) (layer "F.Cu") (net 32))
 (segment (start 148.585 90.18) (end 148.585 96.515) (width 0.2) (layer "F.Cu") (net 32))
 (segment (start 146.045 95.245) (end 146.045 90.18) (width 0.2) (layer "F.Cu") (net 31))
 (segment (start 146.05 96.52) (end 146.05 95.25) (width 0.2) (layer "F.Cu") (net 31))
 (segment (start 146.05 95.25) (end 146.045 95.245) (width 0.2) (layer "F.Cu") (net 31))
 (segment (start 143.505 90.18) (end 143.505 96.515) (width 0.2) (layer "F.Cu") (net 30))
 (segment (start 143.505 96.515) (end 143.51 96.52) (width 0.2) (layer "F.Cu") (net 30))
 (segment (start 140.97 96.52) (end 140.97 90.185) (width 0.2) (layer "F.Cu") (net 29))
 (segment (start 140.97 90.185) (end 140.965 90.18) (width 0.2) (layer "F.Cu") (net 29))
 (segment (start 138.425 95.245) (end 138.43 95.25) (width 0.2) (layer "F.Cu") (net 28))
 (segment (start 138.425 90.18) (end 138.425 95.245) (width 0.2) (layer "F.Cu") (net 28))
 (segment (start 138.43 95.25) (end 138.43 96.52) (width 0.2) (layer "F.Cu") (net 28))
 (segment (start 135.89 96.52) (end 135.89 95.25) (width 0.2) (layer "F.Cu") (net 27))
 (segment (start 135.89 95.25) (end 135.885 95.245) (width 0.2) (layer "F.Cu") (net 27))
 (segment (start 135.885 95.245) (end 135.885 90.18) (width 0.2) (layer "F.Cu") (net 27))
 (segment (start 133.35 96.52) (end 133.35 95.25) (width 0.2) (layer "F.Cu") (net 26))
 (segment (start 133.345 95.245) (end 133.345 90.18) (width 0.2) (layer "F.Cu") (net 26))
 (segment (start 133.35 95.25) (end 133.345 95.245) (width 0.2) (layer "F.Cu") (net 26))
 (segment (start 158.496 115.316) (end 168.656 115.316) (width 0.2) (layer "F.Cu") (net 35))
 (segment (start 151.13 106.68) (end 151.13 107.95) (width 0.2) (layer "F.Cu") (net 35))
 (segment (start 151.13 107.95) (end 158.496 115.316) (width 0.2) (layer "F.Cu") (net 35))
 (segment (start 168.656 115.316) (end 170.18 116.84) (width 0.2) (layer "F.Cu") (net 35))
 (segment (start 158.75 102.87) (end 151.13 102.87) (width 0.2) (layer "F.Cu") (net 41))
 (segment (start 148.59 105.41) (end 148.59 106.68) (width 0.2) (layer "F.Cu") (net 41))
 (segment (start 151.13 102.87) (end 148.59 105.41) (width 0.2) (layer "F.Cu") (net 41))
 (segment (start 160.02 101.6) (end 158.75 102.87) (width 0.2) (layer "F.Cu") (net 41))
 (segment (start 151.13 104.14) (end 149.86 105.41) (width 0.2) (layer "F.Cu") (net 36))
 (segment (start 149.86 105.41) (end 149.86 107.696) (width 0.2) (layer "F.Cu") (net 36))
 (segment (start 146.558 106.68) (end 146.05 106.68) (width 0.2) (layer "F.Cu") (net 36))
 (segment (start 162.56 101.6) (end 160.02 104.14) (width 0.2) (layer "F.Cu") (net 36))
 (segment (start 149.098 108.458) (end 146.812 108.458) (width 0.2) (layer "F.Cu") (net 36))
 (segment (start 149.86 107.696) (end 149.098 108.458) (width 0.2) (layer "F.Cu") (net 36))
 (segment (start 160.02 104.14) (end 151.13 104.14) (width 0.2) (layer "F.Cu") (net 36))
 (segment (start 146.812 108.458) (end 146.05 107.696) (width 0.2) (layer "F.Cu") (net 36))
 (segment (start 146.05 107.696) (end 146.05 106.68) (width 0.2) (layer "F.Cu") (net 36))
 (segment (start 160.02 116.84) (end 152.4 116.84) (width 0.2) (layer "F.Cu") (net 39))
 (segment (start 152.4 116.84) (end 143.51 107.95) (width 0.2) (layer "F.Cu") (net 39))
 (segment (start 143.51 107.95) (end 143.51 106.68) (width 0.2) (layer "F.Cu") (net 39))
 (segment (start 140.97 106.68) (end 140.97 108.077) (width 0.2) (layer "F.Cu") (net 37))
 (segment (start 151.003 118.11) (end 161.29 118.11) (width 0.2) (layer "F.Cu") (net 37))
 (segment (start 140.97 108.077) (end 151.003 118.11) (width 0.2) (layer "F.Cu") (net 37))
 (segment (start 161.29 118.11) (end 162.56 116.84) (width 0.2) (layer "F.Cu") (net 37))
 (segment (start 138.43 107.95) (end 149.86 119.38) (width 0.2) (layer "F.Cu") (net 34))
 (segment (start 149.86 119.38) (end 165.1 119.38) (width 0.2) (layer "F.Cu") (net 34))
 (segment (start 138.43 106.68) (end 138.43 107.95) (width 0.2) (layer "F.Cu") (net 34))
 (segment (start 165.1 119.38) (end 167.64 116.84) (width 0.2) (layer "F.Cu") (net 34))
 (segment (start 167.64 99.06) (end 142.24 99.06) (width 0.2) (layer "F.Cu") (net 38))
 (segment (start 142.24 99.06) (end 135.89 105.41) (width 0.2) (layer "F.Cu") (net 38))
 (segment (start 135.89 105.41) (end 135.89 106.68) (width 0.2) (layer "F.Cu") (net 38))
 (segment (start 170.18 101.6) (end 167.64 99.06) (width 0.2) (layer "F.Cu") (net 38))
 (segment (start 166.37 100.33) (end 142.24 100.33) (width 0.2) (layer "F.Cu") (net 40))
 (segment (start 133.35 107.696) (end 133.35 106.68) (width 0.2) (layer "F.Cu") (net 40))
 (segment (start 136.398 108.458) (end 134.112 108.458) (width 0.2) (layer "F.Cu") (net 40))
 (segment (start 137.16 105.41) (end 137.16 107.696) (width 0.2) (layer "F.Cu") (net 40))
 (segment (start 142.24 100.33) (end 137.16 105.41) (width 0.2) (layer "F.Cu") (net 40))
 (segment (start 167.64 101.6) (end 166.37 100.33) (width 0.2) (layer "F.Cu") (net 40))
 (segment (start 134.112 108.458) (end 133.35 107.696) (width 0.2) (layer "F.Cu") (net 40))
 (segment (start 137.16 107.696) (end 136.398 108.458) (width 0.2) (layer "F.Cu") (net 40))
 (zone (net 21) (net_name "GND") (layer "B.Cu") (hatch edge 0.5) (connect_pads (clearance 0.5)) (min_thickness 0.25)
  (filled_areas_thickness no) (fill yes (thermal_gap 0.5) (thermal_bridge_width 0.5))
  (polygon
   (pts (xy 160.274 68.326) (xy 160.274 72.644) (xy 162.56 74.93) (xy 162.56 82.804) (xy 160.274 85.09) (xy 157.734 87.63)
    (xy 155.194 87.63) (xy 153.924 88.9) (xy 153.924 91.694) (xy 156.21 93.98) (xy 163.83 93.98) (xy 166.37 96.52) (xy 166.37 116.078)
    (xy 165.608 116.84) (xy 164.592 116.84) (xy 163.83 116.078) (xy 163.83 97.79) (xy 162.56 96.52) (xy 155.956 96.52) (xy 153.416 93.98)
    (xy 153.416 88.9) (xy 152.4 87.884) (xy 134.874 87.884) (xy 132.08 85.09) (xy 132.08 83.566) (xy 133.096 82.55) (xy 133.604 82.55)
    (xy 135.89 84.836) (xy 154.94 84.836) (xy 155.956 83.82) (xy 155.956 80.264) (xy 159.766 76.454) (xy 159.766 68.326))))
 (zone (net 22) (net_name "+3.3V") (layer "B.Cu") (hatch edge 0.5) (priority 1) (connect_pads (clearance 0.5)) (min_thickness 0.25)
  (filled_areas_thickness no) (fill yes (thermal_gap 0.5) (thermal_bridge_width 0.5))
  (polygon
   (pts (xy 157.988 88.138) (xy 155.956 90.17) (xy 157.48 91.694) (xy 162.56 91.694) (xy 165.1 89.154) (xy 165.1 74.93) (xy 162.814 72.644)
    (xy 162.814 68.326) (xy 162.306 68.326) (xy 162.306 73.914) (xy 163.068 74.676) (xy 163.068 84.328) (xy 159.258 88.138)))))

